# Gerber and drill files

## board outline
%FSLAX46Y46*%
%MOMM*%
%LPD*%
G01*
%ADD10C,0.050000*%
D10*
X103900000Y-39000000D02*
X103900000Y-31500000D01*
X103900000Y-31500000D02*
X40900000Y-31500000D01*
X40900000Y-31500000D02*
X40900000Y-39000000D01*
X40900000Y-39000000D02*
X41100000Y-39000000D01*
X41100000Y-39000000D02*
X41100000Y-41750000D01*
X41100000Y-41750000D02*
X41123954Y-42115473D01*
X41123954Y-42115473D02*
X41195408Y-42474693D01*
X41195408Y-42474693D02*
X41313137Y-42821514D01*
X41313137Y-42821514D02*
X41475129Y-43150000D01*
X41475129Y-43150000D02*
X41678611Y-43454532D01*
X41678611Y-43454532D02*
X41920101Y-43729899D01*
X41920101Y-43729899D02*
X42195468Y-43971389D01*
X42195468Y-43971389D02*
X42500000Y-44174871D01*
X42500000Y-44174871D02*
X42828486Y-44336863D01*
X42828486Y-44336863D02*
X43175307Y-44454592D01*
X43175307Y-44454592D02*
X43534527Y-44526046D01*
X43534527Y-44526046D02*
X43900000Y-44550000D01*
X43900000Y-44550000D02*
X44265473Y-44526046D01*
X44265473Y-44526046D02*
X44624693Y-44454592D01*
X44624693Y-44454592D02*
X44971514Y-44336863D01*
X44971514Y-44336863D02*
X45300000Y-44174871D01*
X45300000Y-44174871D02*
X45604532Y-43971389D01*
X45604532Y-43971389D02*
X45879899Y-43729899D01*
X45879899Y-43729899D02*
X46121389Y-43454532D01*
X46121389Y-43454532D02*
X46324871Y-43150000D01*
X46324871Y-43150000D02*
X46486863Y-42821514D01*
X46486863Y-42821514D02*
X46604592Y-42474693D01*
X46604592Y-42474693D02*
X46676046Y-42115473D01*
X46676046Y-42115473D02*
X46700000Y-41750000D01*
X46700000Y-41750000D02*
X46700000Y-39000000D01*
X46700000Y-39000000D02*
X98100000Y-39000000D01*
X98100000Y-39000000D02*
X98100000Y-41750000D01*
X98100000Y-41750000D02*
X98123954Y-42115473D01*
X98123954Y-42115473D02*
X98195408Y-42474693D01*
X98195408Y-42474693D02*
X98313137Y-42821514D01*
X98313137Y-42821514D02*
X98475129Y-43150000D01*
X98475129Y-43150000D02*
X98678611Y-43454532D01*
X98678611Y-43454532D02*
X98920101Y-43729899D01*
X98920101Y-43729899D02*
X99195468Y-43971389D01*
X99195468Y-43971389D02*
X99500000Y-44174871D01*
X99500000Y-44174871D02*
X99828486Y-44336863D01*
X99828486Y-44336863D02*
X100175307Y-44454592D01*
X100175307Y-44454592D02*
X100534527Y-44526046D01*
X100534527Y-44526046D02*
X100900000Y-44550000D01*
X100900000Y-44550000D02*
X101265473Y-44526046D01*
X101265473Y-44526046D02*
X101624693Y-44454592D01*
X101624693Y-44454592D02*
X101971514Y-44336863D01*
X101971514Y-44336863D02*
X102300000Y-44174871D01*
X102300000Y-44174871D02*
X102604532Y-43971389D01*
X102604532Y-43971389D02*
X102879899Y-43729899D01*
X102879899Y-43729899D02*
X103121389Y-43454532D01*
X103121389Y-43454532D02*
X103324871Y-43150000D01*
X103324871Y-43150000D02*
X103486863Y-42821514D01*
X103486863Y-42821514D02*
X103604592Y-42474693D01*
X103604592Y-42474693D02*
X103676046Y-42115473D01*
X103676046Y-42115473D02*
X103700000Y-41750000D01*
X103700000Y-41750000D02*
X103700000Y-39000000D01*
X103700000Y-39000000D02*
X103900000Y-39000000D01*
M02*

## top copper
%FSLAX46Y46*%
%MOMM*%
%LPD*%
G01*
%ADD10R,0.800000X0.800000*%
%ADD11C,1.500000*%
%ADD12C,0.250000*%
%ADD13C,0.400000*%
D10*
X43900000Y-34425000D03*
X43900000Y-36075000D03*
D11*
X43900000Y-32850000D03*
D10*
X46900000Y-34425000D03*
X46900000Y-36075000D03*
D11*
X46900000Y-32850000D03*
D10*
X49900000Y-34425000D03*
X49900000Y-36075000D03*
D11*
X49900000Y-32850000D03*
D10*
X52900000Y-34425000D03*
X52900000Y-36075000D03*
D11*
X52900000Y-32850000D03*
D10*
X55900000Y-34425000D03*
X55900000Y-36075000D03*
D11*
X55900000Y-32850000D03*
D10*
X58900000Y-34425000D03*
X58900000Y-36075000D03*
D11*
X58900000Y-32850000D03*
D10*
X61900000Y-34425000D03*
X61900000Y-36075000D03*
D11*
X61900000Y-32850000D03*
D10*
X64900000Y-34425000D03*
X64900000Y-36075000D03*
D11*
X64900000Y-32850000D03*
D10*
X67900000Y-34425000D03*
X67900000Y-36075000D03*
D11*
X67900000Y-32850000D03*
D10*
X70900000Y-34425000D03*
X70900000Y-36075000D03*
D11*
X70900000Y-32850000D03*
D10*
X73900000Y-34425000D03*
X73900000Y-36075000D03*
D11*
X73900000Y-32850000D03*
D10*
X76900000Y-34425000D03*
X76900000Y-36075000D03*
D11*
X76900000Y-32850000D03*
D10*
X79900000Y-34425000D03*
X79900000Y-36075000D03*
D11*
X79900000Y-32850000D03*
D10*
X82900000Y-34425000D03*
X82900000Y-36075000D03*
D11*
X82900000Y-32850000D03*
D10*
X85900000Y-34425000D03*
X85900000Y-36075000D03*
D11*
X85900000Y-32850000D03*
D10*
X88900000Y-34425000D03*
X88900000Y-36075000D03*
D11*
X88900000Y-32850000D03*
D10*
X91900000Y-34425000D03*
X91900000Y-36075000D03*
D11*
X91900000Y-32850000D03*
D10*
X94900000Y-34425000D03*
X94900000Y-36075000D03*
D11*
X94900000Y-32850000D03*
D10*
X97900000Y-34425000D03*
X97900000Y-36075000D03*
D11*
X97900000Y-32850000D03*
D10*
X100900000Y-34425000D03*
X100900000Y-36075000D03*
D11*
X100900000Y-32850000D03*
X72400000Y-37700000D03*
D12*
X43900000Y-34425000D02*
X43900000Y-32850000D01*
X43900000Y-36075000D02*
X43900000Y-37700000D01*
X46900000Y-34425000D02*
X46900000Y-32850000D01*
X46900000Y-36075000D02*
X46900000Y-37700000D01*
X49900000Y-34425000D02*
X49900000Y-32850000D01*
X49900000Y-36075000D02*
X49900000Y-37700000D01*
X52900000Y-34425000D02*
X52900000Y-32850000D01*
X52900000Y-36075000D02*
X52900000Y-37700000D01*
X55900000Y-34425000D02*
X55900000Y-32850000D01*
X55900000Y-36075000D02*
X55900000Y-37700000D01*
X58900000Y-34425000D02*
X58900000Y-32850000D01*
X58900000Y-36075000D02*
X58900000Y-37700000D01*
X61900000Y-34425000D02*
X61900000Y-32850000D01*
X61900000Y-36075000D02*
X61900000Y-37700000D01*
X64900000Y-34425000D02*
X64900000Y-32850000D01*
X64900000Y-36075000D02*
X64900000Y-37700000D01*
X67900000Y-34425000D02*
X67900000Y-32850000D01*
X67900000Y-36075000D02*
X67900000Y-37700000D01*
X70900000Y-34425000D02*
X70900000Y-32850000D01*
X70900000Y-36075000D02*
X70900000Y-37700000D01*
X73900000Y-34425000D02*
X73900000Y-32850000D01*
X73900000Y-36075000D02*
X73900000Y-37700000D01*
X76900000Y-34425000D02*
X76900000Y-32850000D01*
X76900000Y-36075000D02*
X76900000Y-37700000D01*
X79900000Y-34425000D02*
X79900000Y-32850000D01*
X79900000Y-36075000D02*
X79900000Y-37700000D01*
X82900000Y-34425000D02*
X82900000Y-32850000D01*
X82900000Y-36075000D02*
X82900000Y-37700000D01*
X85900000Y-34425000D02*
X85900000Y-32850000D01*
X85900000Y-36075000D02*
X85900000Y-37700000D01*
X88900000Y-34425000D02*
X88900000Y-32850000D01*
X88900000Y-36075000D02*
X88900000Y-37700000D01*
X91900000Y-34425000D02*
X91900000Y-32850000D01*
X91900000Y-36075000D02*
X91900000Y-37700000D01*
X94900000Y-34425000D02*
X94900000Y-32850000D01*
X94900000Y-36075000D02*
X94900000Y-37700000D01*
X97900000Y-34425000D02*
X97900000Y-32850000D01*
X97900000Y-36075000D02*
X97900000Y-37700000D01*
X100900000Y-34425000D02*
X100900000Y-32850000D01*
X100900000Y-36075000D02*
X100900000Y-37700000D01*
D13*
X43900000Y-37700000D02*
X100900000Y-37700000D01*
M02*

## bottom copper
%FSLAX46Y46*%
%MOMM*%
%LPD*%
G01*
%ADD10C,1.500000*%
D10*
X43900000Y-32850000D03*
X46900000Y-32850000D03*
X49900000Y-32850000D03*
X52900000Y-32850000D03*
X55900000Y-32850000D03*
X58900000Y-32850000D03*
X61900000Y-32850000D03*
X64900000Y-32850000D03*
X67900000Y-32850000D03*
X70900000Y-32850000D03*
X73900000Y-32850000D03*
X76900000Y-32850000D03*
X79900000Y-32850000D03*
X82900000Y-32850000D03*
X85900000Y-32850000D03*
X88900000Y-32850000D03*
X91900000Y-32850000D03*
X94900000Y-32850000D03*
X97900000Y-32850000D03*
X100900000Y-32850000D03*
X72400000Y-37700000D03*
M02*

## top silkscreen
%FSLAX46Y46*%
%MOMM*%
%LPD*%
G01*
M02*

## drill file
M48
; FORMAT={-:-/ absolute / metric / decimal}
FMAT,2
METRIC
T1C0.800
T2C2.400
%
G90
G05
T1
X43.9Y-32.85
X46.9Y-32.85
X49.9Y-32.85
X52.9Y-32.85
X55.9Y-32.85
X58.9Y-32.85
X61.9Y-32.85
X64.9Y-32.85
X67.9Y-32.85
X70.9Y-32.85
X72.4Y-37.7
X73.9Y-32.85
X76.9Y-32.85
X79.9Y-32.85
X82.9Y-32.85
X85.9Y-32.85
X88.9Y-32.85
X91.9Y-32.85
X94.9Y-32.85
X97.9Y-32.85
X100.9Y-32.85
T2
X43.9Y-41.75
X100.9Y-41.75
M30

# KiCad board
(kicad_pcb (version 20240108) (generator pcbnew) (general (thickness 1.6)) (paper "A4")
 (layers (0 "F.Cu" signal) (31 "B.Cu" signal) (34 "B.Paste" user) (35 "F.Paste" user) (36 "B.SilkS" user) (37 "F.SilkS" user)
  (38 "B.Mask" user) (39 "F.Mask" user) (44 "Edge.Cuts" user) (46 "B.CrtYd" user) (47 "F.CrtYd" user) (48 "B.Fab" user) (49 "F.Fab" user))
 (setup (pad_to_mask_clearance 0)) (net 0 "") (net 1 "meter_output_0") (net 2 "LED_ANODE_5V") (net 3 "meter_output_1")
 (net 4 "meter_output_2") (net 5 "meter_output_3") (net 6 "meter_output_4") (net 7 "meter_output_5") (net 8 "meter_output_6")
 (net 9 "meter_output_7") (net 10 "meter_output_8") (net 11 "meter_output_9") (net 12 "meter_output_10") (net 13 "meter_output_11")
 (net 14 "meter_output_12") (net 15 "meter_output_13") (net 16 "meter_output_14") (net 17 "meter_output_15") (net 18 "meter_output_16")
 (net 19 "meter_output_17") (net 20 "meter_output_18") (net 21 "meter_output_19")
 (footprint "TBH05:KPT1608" (layer "F.Cu") (at 43.9 35.25)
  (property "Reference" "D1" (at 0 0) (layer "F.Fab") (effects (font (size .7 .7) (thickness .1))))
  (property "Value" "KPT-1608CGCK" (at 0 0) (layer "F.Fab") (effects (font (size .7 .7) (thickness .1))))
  (pad "1" smd rect (at 0 -.825) (size .8 .8) (layers "F.Cu" "F.Paste" "F.Mask") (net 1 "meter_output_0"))
  (pad "2" smd rect (at 0 .825) (size .8 .8) (layers "F.Cu" "F.Paste" "F.Mask") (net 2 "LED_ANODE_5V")))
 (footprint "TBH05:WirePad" (layer "F.Cu") (at 43.9 32.85)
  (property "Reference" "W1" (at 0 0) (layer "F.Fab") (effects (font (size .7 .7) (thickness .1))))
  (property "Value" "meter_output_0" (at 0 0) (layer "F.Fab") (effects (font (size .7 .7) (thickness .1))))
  (pad "1" thru_hole circle (at 0 0) (size 1.5 1.5) (drill .8) (layers "*.Cu" "*.Mask") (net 1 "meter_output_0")))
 (segment (start 43.9 34.425) (end 43.9 32.85) (width 0.25) (layer "F.Cu") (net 1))
 (segment (start 43.9 36.075) (end 43.9 37.7) (width 0.25) (layer "F.Cu") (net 2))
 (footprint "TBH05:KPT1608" (layer "F.Cu") (at 46.9 35.25)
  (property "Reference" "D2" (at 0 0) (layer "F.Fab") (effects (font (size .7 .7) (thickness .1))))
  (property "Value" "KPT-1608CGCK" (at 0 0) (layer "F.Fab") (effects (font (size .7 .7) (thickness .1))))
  (pad "1" smd rect (at 0 -.825) (size .8 .8) (layers "F.Cu" "F.Paste" "F.Mask") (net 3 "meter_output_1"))
  (pad "2" smd rect (at 0 .825) (size .8 .8) (layers "F.Cu" "F.Paste" "F.Mask") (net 2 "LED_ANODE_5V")))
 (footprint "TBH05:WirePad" (layer "F.Cu") (at 46.9 32.85)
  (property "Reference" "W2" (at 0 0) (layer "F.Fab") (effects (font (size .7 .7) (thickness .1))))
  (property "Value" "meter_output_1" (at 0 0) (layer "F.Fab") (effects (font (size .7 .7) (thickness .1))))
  (pad "1" thru_hole circle (at 0 0) (size 1.5 1.5) (drill .8) (layers "*.Cu" "*.Mask") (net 3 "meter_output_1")))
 (segment (start 46.9 34.425) (end 46.9 32.85) (width 0.25) (layer "F.Cu") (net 3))
 (segment (start 46.9 36.075) (end 46.9 37.7) (width 0.25) (layer "F.Cu") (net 2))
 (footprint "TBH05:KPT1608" (layer "F.Cu") (at 49.9 35.25)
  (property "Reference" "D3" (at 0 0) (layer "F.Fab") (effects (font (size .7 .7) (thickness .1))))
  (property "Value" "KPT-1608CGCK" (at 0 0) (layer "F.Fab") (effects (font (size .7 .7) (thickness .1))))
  (pad "1" smd rect (at 0 -.825) (size .8 .8) (layers "F.Cu" "F.Paste" "F.Mask") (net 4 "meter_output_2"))
  (pad "2" smd rect (at 0 .825) (size .8 .8) (layers "F.Cu" "F.Paste" "F.Mask") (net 2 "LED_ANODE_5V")))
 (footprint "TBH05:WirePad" (layer "F.Cu") (at 49.9 32.85)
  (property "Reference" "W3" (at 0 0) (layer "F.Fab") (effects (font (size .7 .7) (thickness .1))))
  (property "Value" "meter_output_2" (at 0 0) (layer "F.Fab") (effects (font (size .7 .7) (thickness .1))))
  (pad "1" thru_hole circle (at 0 0) (size 1.5 1.5) (drill .8) (layers "*.Cu" "*.Mask") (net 4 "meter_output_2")))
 (segment (start 49.9 34.425) (end 49.9 32.85) (width 0.25) (layer "F.Cu") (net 4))
 (segment (start 49.9 36.075) (end 49.9 37.7) (width 0.25) (layer "F.Cu") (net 2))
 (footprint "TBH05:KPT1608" (layer "F.Cu") (at 52.9 35.25)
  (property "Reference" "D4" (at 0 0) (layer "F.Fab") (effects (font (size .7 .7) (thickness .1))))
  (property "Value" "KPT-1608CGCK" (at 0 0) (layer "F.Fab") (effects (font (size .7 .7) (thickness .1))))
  (pad "1" smd rect (at 0 -.825) (size .8 .8) (layers "F.Cu" "F.Paste" "F.Mask") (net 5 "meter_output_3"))
  (pad "2" smd rect (at 0 .825) (size .8 .8) (layers "F.Cu" "F.Paste" "F.Mask") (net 2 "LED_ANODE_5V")))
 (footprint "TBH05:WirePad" (layer "F.Cu") (at 52.9 32.85)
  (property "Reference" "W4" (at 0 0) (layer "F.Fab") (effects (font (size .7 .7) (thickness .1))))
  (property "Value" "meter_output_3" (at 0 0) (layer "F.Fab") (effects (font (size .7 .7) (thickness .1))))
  (pad "1" thru_hole circle (at 0 0) (size 1.5 1.5) (drill .8) (layers "*.Cu" "*.Mask") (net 5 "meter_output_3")))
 (segment (start 52.9 34.425) (end 52.9 32.85) (width 0.25) (layer "F.Cu") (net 5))
 (segment (start 52.9 36.075) (end 52.9 37.7) (width 0.25) (layer "F.Cu") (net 2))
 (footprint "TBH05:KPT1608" (layer "F.Cu") (at 55.9 35.25)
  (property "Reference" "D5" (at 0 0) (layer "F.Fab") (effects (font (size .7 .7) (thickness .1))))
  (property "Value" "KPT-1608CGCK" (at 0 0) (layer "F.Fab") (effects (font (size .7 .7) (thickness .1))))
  (pad "1" smd rect (at 0 -.825) (size .8 .8) (layers "F.Cu" "F.Paste" "F.Mask") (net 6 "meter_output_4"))
  (pad "2" smd rect (at 0 .825) (size .8 .8) (layers "F.Cu" "F.Paste" "F.Mask") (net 2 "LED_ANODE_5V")))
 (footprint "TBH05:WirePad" (layer "F.Cu") (at 55.9 32.85)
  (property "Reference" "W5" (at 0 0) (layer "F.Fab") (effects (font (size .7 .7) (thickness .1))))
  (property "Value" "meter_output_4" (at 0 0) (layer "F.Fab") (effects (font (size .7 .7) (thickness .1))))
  (pad "1" thru_hole circle (at 0 0) (size 1.5 1.5) (drill .8) (layers "*.Cu" "*.Mask") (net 6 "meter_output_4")))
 (segment (start 55.9 34.425) (end 55.9 32.85) (width 0.25) (layer "F.Cu") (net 6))
 (segment (start 55.9 36.075) (end 55.9 37.7) (width 0.25) (layer "F.Cu") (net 2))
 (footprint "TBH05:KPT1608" (layer "F.Cu") (at 58.9 35.25)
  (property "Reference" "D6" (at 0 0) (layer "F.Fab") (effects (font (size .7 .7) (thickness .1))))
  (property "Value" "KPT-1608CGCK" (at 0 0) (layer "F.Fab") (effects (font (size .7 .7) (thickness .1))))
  (pad "1" smd rect (at 0 -.825) (size .8 .8) (layers "F.Cu" "F.Paste" "F.Mask") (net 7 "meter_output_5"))
  (pad "2" smd rect (at 0 .825) (size .8 .8) (layers "F.Cu" "F.Paste" "F.Mask") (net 2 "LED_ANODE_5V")))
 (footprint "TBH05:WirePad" (layer "F.Cu") (at 58.9 32.85)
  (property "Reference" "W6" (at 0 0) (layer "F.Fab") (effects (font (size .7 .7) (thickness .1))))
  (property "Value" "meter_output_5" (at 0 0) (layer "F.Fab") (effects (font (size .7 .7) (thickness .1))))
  (pad "1" thru_hole circle (at 0 0) (size 1.5 1.5) (drill .8) (layers "*.Cu" "*.Mask") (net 7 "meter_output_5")))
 (segment (start 58.9 34.425) (end 58.9 32.85) (width 0.25) (layer "F.Cu") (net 7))
 (segment (start 58.9 36.075) (end 58.9 37.7) (width 0.25) (layer "F.Cu") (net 2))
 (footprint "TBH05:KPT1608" (layer "F.Cu") (at 61.9 35.25)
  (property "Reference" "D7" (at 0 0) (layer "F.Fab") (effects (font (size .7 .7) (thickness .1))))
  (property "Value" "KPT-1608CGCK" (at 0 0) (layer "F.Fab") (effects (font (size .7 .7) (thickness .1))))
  (pad "1" smd rect (at 0 -.825) (size .8 .8) (layers "F.Cu" "F.Paste" "F.Mask") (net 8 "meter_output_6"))
  (pad "2" smd rect (at 0 .825) (size .8 .8) (layers "F.Cu" "F.Paste" "F.Mask") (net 2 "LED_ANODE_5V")))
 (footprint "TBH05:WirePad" (layer "F.Cu") (at 61.9 32.85)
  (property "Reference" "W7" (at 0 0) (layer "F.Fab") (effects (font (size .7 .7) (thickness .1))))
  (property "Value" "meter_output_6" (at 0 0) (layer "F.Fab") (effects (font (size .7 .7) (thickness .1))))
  (pad "1" thru_hole circle (at 0 0) (size 1.5 1.5) (drill .8) (layers "*.Cu" "*.Mask") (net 8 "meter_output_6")))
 (segment (start 61.9 34.425) (end 61.9 32.85) (width 0.25) (layer "F.Cu") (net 8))
 (segment (start 61.9 36.075) (end 61.9 37.7) (width 0.25) (layer "F.Cu") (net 2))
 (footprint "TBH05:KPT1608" (layer "F.Cu") (at 64.9 35.25)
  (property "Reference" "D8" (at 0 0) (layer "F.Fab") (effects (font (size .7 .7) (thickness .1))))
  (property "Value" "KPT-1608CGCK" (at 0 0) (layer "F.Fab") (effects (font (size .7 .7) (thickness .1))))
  (pad "1" smd rect (at 0 -.825) (size .8 .8) (layers "F.Cu" "F.Paste" "F.Mask") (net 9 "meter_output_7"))
  (pad "2" smd rect (at 0 .825) (size .8 .8) (layers "F.Cu" "F.Paste" "F.Mask") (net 2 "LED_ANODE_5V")))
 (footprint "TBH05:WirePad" (layer "F.Cu") (at 64.9 32.85)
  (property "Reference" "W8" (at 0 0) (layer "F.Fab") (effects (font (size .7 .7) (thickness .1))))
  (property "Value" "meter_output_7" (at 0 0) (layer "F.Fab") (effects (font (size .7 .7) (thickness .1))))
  (pad "1" thru_hole circle (at 0 0) (size 1.5 1.5) (drill .8) (layers "*.Cu" "*.Mask") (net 9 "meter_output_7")))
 (segment (start 64.9 34.425) (end 64.9 32.85) (width 0.25) (layer "F.Cu") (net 9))
 (segment (start 64.9 36.075) (end 64.9 37.7) (width 0.25) (layer "F.Cu") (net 2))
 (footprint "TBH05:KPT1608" (layer "F.Cu") (at 67.9 35.25)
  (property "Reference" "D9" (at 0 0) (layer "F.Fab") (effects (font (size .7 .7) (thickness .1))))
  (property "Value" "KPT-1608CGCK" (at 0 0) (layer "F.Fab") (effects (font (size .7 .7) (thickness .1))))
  (pad "1" smd rect (at 0 -.825) (size .8 .8) (layers "F.Cu" "F.Paste" "F.Mask") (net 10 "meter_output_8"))
  (pad "2" smd rect (at 0 .825) (size .8 .8) (layers "F.Cu" "F.Paste" "F.Mask") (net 2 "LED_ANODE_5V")))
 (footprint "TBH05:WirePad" (layer "F.Cu") (at 67.9 32.85)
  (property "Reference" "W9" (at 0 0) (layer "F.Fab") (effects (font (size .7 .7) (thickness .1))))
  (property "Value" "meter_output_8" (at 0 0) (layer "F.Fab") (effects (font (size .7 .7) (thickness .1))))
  (pad "1" thru_hole circle (at 0 0) (size 1.5 1.5) (drill .8) (layers "*.Cu" "*.Mask") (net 10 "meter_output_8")))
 (segment (start 67.9 34.425) (end 67.9 32.85) (width 0.25) (layer "F.Cu") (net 10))
 (segment (start 67.9 36.075) (end 67.9 37.7) (width 0.25) (layer "F.Cu") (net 2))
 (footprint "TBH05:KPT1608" (layer "F.Cu") (at 70.9 35.25)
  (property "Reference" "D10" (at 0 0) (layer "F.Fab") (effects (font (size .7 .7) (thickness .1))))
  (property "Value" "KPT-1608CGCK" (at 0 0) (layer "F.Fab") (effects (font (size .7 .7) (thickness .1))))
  (pad "1" smd rect (at 0 -.825) (size .8 .8) (layers "F.Cu" "F.Paste" "F.Mask") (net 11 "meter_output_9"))
  (pad "2" smd rect (at 0 .825) (size .8 .8) (layers "F.Cu" "F.Paste" "F.Mask") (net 2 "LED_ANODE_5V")))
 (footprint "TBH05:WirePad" (layer "F.Cu") (at 70.9 32.85)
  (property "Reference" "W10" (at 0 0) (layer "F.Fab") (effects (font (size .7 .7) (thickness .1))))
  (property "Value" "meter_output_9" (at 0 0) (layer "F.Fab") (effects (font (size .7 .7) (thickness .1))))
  (pad "1" thru_hole circle (at 0 0) (size 1.5 1.5) (drill .8) (layers "*.Cu" "*.Mask") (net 11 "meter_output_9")))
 (segment (start 70.9 34.425) (end 70.9 32.85) (width 0.25) (layer "F.Cu") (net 11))
 (segment (start 70.9 36.075) (end 70.9 37.7) (width 0.25) (layer "F.Cu") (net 2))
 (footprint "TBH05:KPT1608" (layer "F.Cu") (at 73.9 35.25)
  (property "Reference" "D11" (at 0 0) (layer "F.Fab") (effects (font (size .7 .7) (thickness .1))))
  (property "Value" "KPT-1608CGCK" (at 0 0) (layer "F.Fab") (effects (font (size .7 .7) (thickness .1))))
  (pad "1" smd rect (at 0 -.825) (size .8 .8) (layers "F.Cu" "F.Paste" "F.Mask") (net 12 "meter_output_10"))
  (pad "2" smd rect (at 0 .825) (size .8 .8) (layers "F.Cu" "F.Paste" "F.Mask") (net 2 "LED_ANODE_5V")))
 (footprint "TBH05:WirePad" (layer "F.Cu") (at 73.9 32.85)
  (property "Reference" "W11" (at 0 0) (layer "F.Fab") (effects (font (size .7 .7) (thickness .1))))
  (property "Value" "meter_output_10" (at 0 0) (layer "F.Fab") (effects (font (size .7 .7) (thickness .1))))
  (pad "1" thru_hole circle (at 0 0) (size 1.5 1.5) (drill .8) (layers "*.Cu" "*.Mask") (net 12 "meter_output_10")))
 (segment (start 73.9 34.425) (end 73.9 32.85) (width 0.25) (layer "F.Cu") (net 12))
 (segment (start 73.9 36.075) (end 73.9 37.7) (width 0.25) (layer "F.Cu") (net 2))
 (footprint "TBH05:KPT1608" (layer "F.Cu") (at 76.9 35.25)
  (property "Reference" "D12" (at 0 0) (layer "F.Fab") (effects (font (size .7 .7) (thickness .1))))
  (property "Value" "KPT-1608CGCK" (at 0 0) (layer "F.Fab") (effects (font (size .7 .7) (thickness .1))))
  (pad "1" smd rect (at 0 -.825) (size .8 .8) (layers "F.Cu" "F.Paste" "F.Mask") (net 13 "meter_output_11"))
  (pad "2" smd rect (at 0 .825) (size .8 .8) (layers "F.Cu" "F.Paste" "F.Mask") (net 2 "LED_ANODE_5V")))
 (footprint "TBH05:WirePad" (layer "F.Cu") (at 76.9 32.85)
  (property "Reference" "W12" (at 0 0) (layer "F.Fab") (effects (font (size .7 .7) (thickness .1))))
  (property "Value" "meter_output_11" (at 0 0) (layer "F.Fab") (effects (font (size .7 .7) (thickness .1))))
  (pad "1" thru_hole circle (at 0 0) (size 1.5 1.5) (drill .8) (layers "*.Cu" "*.Mask") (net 13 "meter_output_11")))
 (segment (start 76.9 34.425) (end 76.9 32.85) (width 0.25) (layer "F.Cu") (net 13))
 (segment (start 76.9 36.075) (end 76.9 37.7) (width 0.25) (layer "F.Cu") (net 2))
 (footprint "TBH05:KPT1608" (layer "F.Cu") (at 79.9 35.25)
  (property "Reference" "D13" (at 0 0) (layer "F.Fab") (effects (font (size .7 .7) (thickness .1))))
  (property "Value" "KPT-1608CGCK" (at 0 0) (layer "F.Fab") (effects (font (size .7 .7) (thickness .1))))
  (pad "1" smd rect (at 0 -.825) (size .8 .8) (layers "F.Cu" "F.Paste" "F.Mask") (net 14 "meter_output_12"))
  (pad "2" smd rect (at 0 .825) (size .8 .8) (layers "F.Cu" "F.Paste" "F.Mask") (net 2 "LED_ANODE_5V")))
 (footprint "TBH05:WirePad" (layer "F.Cu") (at 79.9 32.85)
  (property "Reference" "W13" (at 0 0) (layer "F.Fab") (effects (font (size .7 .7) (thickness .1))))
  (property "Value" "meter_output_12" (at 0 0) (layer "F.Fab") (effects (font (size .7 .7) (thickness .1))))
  (pad "1" thru_hole circle (at 0 0) (size 1.5 1.5) (drill .8) (layers "*.Cu" "*.Mask") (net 14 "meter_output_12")))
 (segment (start 79.9 34.425) (end 79.9 32.85) (width 0.25) (layer "F.Cu") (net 14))
 (segment (start 79.9 36.075) (end 79.9 37.7) (width 0.25) (layer "F.Cu") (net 2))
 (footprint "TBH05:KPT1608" (layer "F.Cu") (at 82.9 35.25)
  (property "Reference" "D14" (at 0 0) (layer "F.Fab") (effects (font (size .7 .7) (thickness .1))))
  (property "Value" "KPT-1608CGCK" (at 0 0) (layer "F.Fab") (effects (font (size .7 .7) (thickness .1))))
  (pad "1" smd rect (at 0 -.825) (size .8 .8) (layers "F.Cu" "F.Paste" "F.Mask") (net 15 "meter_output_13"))
  (pad "2" smd rect (at 0 .825) (size .8 .8) (layers "F.Cu" "F.Paste" "F.Mask") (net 2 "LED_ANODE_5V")))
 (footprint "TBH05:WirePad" (layer "F.Cu") (at 82.9 32.85)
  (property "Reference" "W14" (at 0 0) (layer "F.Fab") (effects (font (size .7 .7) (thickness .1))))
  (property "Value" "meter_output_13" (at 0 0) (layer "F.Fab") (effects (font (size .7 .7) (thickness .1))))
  (pad "1" thru_hole circle (at 0 0) (size 1.5 1.5) (drill .8) (layers "*.Cu" "*.Mask") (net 15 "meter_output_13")))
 (segment (start 82.9 34.425) (end 82.9 32.85) (width 0.25) (layer "F.Cu") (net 15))
 (segment (start 82.9 36.075) (end 82.9 37.7) (width 0.25) (layer "F.Cu") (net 2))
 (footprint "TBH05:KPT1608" (layer "F.Cu") (at 85.9 35.25)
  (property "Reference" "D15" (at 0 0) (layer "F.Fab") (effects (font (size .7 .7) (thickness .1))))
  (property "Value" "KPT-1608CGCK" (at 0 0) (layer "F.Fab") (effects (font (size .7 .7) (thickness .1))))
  (pad "1" smd rect (at 0 -.825) (size .8 .8) (layers "F.Cu" "F.Paste" "F.Mask") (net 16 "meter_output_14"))
  (pad "2" smd rect (at 0 .825) (size .8 .8) (layers "F.Cu" "F.Paste" "F.Mask") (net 2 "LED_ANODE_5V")))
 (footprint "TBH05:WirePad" (layer "F.Cu") (at 85.9 32.85)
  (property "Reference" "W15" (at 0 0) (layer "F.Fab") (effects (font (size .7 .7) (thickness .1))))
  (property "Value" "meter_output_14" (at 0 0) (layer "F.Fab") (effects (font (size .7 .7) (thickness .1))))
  (pad "1" thru_hole circle (at 0 0) (size 1.5 1.5) (drill .8) (layers "*.Cu" "*.Mask") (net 16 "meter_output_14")))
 (segment (start 85.9 34.425) (end 85.9 32.85) (width 0.25) (layer "F.Cu") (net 16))
 (segment (start 85.9 36.075) (end 85.9 37.7) (width 0.25) (layer "F.Cu") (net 2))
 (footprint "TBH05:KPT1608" (layer "F.Cu") (at 88.9 35.25)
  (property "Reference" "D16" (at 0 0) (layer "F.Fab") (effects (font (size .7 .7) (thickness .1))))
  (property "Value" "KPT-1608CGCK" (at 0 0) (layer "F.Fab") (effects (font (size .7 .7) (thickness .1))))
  (pad "1" smd rect (at 0 -.825) (size .8 .8) (layers "F.Cu" "F.Paste" "F.Mask") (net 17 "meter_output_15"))
  (pad "2" smd rect (at 0 .825) (size .8 .8) (layers "F.Cu" "F.Paste" "F.Mask") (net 2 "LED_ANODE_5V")))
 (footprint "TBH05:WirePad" (layer "F.Cu") (at 88.9 32.85)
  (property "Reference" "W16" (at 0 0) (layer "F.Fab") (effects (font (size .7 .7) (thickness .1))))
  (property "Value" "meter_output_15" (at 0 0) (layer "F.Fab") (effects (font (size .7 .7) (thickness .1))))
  (pad "1" thru_hole circle (at 0 0) (size 1.5 1.5) (drill .8) (layers "*.Cu" "*.Mask") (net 17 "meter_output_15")))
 (segment (start 88.9 34.425) (end 88.9 32.85) (width 0.25) (layer "F.Cu") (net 17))
 (segment (start 88.9 36.075) (end 88.9 37.7) (width 0.25) (layer "F.Cu") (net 2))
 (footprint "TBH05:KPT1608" (layer "F.Cu") (at 91.9 35.25)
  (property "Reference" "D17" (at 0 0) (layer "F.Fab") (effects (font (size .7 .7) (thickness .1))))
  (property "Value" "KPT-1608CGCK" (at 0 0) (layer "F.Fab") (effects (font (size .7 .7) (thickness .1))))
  (pad "1" smd rect (at 0 -.825) (size .8 .8) (layers "F.Cu" "F.Paste" "F.Mask") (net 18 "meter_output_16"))
  (pad "2" smd rect (at 0 .825) (size .8 .8) (layers "F.Cu" "F.Paste" "F.Mask") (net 2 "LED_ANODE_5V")))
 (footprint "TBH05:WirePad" (layer "F.Cu") (at 91.9 32.85)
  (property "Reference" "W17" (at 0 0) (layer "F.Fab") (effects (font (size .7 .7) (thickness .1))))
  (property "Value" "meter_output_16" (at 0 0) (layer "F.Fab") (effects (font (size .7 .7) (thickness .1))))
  (pad "1" thru_hole circle (at 0 0) (size 1.5 1.5) (drill .8) (layers "*.Cu" "*.Mask") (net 18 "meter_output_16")))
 (segment (start 91.9 34.425) (end 91.9 32.85) (width 0.25) (layer "F.Cu") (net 18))
 (segment (start 91.9 36.075) (end 91.9 37.7) (width 0.25) (layer "F.Cu") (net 2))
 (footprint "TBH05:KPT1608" (layer "F.Cu") (at 94.9 35.25)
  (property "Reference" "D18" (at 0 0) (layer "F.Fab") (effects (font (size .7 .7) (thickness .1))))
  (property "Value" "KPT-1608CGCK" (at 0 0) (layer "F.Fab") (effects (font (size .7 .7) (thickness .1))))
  (pad "1" smd rect (at 0 -.825) (size .8 .8) (layers "F.Cu" "F.Paste" "F.Mask") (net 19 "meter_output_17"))
  (pad "2" smd rect (at 0 .825) (size .8 .8) (layers "F.Cu" "F.Paste" "F.Mask") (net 2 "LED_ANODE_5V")))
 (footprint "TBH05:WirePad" (layer "F.Cu") (at 94.9 32.85)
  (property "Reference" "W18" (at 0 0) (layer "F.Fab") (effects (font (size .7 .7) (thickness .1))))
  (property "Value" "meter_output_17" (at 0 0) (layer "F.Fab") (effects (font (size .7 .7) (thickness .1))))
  (pad "1" thru_hole circle (at 0 0) (size 1.5 1.5) (drill .8) (layers "*.Cu" "*.Mask") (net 19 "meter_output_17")))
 (segment (start 94.9 34.425) (end 94.9 32.85) (width 0.25) (layer "F.Cu") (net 19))
 (segment (start 94.9 36.075) (end 94.9 37.7) (width 0.25) (layer "F.Cu") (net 2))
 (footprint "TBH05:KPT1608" (layer "F.Cu") (at 97.9 35.25)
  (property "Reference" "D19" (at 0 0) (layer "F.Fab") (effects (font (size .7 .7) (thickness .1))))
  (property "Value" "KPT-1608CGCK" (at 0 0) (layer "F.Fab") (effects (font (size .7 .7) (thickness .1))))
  (pad "1" smd rect (at 0 -.825) (size .8 .8) (layers "F.Cu" "F.Paste" "F.Mask") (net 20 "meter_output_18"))
  (pad "2" smd rect (at 0 .825) (size .8 .8) (layers "F.Cu" "F.Paste" "F.Mask") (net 2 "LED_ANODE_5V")))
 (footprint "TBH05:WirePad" (layer "F.Cu") (at 97.9 32.85)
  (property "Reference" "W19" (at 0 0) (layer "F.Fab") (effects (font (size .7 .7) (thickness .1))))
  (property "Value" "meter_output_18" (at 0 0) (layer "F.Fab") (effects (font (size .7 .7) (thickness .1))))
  (pad "1" thru_hole circle (at 0 0) (size 1.5 1.5) (drill .8) (layers "*.Cu" "*.Mask") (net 20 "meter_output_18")))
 (segment (start 97.9 34.425) (end 97.9 32.85) (width 0.25) (layer "F.Cu") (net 20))
 (segment (start 97.9 36.075) (end 97.9 37.7) (width 0.25) (layer "F.Cu") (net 2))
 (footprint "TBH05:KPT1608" (layer "F.Cu") (at 100.9 35.25)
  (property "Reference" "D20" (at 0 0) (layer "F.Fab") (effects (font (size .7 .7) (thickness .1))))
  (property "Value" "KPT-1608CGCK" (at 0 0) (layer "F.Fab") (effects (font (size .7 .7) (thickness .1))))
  (pad "1" smd rect (at 0 -.825) (size .8 .8) (layers "F.Cu" "F.Paste" "F.Mask") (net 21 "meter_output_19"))
  (pad "2" smd rect (at 0 .825) (size .8 .8) (layers "F.Cu" "F.Paste" "F.Mask") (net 2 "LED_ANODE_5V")))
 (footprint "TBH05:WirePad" (layer "F.Cu") (at 100.9 32.85)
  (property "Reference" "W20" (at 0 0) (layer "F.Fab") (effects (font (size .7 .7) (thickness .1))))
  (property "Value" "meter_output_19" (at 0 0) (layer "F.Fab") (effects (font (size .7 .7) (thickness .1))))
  (pad "1" thru_hole circle (at 0 0) (size 1.5 1.5) (drill .8) (layers "*.Cu" "*.Mask") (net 21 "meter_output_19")))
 (segment (start 100.9 34.425) (end 100.9 32.85) (width 0.25) (layer "F.Cu") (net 21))
 (segment (start 100.9 36.075) (end 100.9 37.7) (width 0.25) (layer "F.Cu") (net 2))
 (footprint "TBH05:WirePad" (layer "F.Cu") (at 72.4 37.7)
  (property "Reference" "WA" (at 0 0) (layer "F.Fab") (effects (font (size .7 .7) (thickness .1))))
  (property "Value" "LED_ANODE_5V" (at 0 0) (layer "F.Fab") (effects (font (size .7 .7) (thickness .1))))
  (pad "1" thru_hole circle (at 0 0) (size 1.5 1.5) (drill .8) (layers "*.Cu" "*.Mask") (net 2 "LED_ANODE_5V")))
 (segment (start 43.9 37.7) (end 100.9 37.7) (width 0.4) (layer "F.Cu") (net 2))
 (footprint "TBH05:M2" (layer "F.Cu") (at 43.9 41.75)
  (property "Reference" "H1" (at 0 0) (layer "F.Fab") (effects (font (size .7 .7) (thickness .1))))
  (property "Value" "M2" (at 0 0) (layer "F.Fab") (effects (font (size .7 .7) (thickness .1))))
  (pad "" np_thru_hole circle (at 0 0) (size 2.4 2.4) (drill 2.4) (layers "*.Cu" "*.Mask")))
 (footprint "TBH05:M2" (layer "F.Cu") (at 100.9 41.75)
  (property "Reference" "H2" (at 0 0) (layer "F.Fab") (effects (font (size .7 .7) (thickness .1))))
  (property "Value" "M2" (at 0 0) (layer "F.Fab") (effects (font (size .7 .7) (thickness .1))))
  (pad "" np_thru_hole circle (at 0 0) (size 2.4 2.4) (drill 2.4) (layers "*.Cu" "*.Mask")))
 (gr_line (start 103.9 39.0) (end 103.9 31.5) (stroke (width .05) (type default)) (layer "Edge.Cuts"))
 (gr_line (start 103.9 31.5) (end 40.9 31.5) (stroke (width .05) (type default)) (layer "Edge.Cuts"))
 (gr_line (start 40.9 31.5) (end 40.9 39.0) (stroke (width .05) (type default)) (layer "Edge.Cuts"))
 (gr_line (start 40.9 39.0) (end 41.1 39.0) (stroke (width .05) (type default)) (layer "Edge.Cuts"))
 (gr_line (start 41.1 39.0) (end 41.1 41.75) (stroke (width .05) (type default)) (layer "Edge.Cuts"))
 (gr_line (start 41.1 41.75) (end 41.123954 42.115473) (stroke (width .05) (type default)) (layer "Edge.Cuts"))
 (gr_line (start 41.123954 42.115473) (end 41.195408 42.474693) (stroke (width .05) (type default)) (layer "Edge.Cuts"))
 (gr_line (start 41.195408 42.474693) (end 41.313137 42.821514) (stroke (width .05) (type default)) (layer "Edge.Cuts"))
 (gr_line (start 41.313137 42.821514) (end 41.475129 43.15) (stroke (width .05) (type default)) (layer "Edge.Cuts"))
 (gr_line (start 41.475129 43.15) (end 41.678611 43.454532) (stroke (width .05) (type default)) (layer "Edge.Cuts"))
 (gr_line (start 41.678611 43.454532) (end 41.920101 43.729899) (stroke (width .05) (type default)) (layer "Edge.Cuts"))
 (gr_line (start 41.920101 43.729899) (end 42.195468 43.971389) (stroke (width .05) (type default)) (layer "Edge.Cuts"))
 (gr_line (start 42.195468 43.971389) (end 42.5 44.174871) (stroke (width .05) (type default)) (layer "Edge.Cuts"))
 (gr_line (start 42.5 44.174871) (end 42.828486 44.336863) (stroke (width .05) (type default)) (layer "Edge.Cuts"))
 (gr_line (start 42.828486 44.336863) (end 43.175307 44.454592) (stroke (width .05) (type default)) (layer "Edge.Cuts"))
 (gr_line (start 43.175307 44.454592) (end 43.534527 44.526046) (stroke (width .05) (type default)) (layer "Edge.Cuts"))
 (gr_line (start 43.534527 44.526046) (end 43.9 44.55) (stroke (width .05) (type default)) (layer "Edge.Cuts"))
 (gr_line (start 43.9 44.55) (end 44.265473 44.526046) (stroke (width .05) (type default)) (layer "Edge.Cuts"))
 (gr_line (start 44.265473 44.526046) (end 44.624693 44.454592) (stroke (width .05) (type default)) (layer "Edge.Cuts"))
 (gr_line (start 44.624693 44.454592) (end 44.971514 44.336863) (stroke (width .05) (type default)) (layer "Edge.Cuts"))
 (gr_line (start 44.971514 44.336863) (end 45.3 44.174871) (stroke (width .05) (type default)) (layer "Edge.Cuts"))
 (gr_line (start 45.3 44.174871) (end 45.604532 43.971389) (stroke (width .05) (type default)) (layer "Edge.Cuts"))
 (gr_line (start 45.604532 43.971389) (end 45.879899 43.729899) (stroke (width .05) (type default)) (layer "Edge.Cuts"))
 (gr_line (start 45.879899 43.729899) (end 46.121389 43.454532) (stroke (width .05) (type default)) (layer "Edge.Cuts"))
 (gr_line (start 46.121389 43.454532) (end 46.324871 43.15) (stroke (width .05) (type default)) (layer "Edge.Cuts"))
 (gr_line (start 46.324871 43.15) (end 46.486863 42.821514) (stroke (width .05) (type default)) (layer "Edge.Cuts"))
 (gr_line (start 46.486863 42.821514) (end 46.604592 42.474693) (stroke (width .05) (type default)) (layer "Edge.Cuts"))
 (gr_line (start 46.604592 42.474693) (end 46.676046 42.115473) (stroke (width .05) (type default)) (layer "Edge.Cuts"))
 (gr_line (start 46.676046 42.115473) (end 46.7 41.75) (stroke (width .05) (type default)) (layer "Edge.Cuts"))
 (gr_line (start 46.7 41.75) (end 46.7 39.0) (stroke (width .05) (type default)) (layer "Edge.Cuts"))
 (gr_line (start 46.7 39.0) (end 98.1 39.0) (stroke (width .05) (type default)) (layer "Edge.Cuts"))
 (gr_line (start 98.1 39.0) (end 98.1 41.75) (stroke (width .05) (type default)) (layer "Edge.Cuts"))
 (gr_line (start 98.1 41.75) (end 98.123954 42.115473) (stroke (width .05) (type default)) (layer "Edge.Cuts"))
 (gr_line (start 98.123954 42.115473) (end 98.195408 42.474693) (stroke (width .05) (type default)) (layer "Edge.Cuts"))
 (gr_line (start 98.195408 42.474693) (end 98.313137 42.821514) (stroke (width .05) (type default)) (layer "Edge.Cuts"))
 (gr_line (start 98.313137 42.821514) (end 98.475129 43.15) (stroke (width .05) (type default)) (layer "Edge.Cuts"))
 (gr_line (start 98.475129 43.15) (end 98.678611 43.454532) (stroke (width .05) (type default)) (layer "Edge.Cuts"))
 (gr_line (start 98.678611 43.454532) (end 98.920101 43.729899) (stroke (width .05) (type default)) (layer "Edge.Cuts"))
 (gr_line (start 98.920101 43.729899) (end 99.195468 43.971389) (stroke (width .05) (type default)) (layer "Edge.Cuts"))
 (gr_line (start 99.195468 43.971389) (end 99.5 44.174871) (stroke (width .05) (type default)) (layer "Edge.Cuts"))
 (gr_line (start 99.5 44.174871) (end 99.828486 44.336863) (stroke (width .05) (type default)) (layer "Edge.Cuts"))
 (gr_line (start 99.828486 44.336863) (end 100.175307 44.454592) (stroke (width .05) (type default)) (layer "Edge.Cuts"))
 (gr_line (start 100.175307 44.454592) (end 100.534527 44.526046) (stroke (width .05) (type default)) (layer "Edge.Cuts"))
 (gr_line (start 100.534527 44.526046) (end 100.9 44.55) (stroke (width .05) (type default)) (layer "Edge.Cuts"))
 (gr_line (start 100.9 44.55) (end 101.265473 44.526046) (stroke (width .05) (type default)) (layer "Edge.Cuts"))
 (gr_line (start 101.265473 44.526046) (end 101.624693 44.454592) (stroke (width .05) (type default)) (layer "Edge.Cuts"))
 (gr_line (start 101.624693 44.454592) (end 101.971514 44.336863) (stroke (width .05) (type default)) (layer "Edge.Cuts"))
 (gr_line (start 101.971514 44.336863) (end 102.3 44.174871) (stroke (width .05) (type default)) (layer "Edge.Cuts"))
 (gr_line (start 102.3 44.174871) (end 102.604532 43.971389) (stroke (width .05) (type default)) (layer "Edge.Cuts"))
 (gr_line (start 102.604532 43.971389) (end 102.879899 43.729899) (stroke (width .05) (type default)) (layer "Edge.Cuts"))
 (gr_line (start 102.879899 43.729899) (end 103.121389 43.454532) (stroke (width .05) (type default)) (layer "Edge.Cuts"))
 (gr_line (start 103.121389 43.454532) (end 103.324871 43.15) (stroke (width .05) (type default)) (layer "Edge.Cuts"))
 (gr_line (start 103.324871 43.15) (end 103.486863 42.821514) (stroke (width .05) (type default)) (layer "Edge.Cuts"))
 (gr_line (start 103.486863 42.821514) (end 103.604592 42.474693) (stroke (width .05) (type default)) (layer "Edge.Cuts"))
 (gr_line (start 103.604592 42.474693) (end 103.676046 42.115473) (stroke (width .05) (type default)) (layer "Edge.Cuts"))
 (gr_line (start 103.676046 42.115473) (end 103.7 41.75) (stroke (width .05) (type default)) (layer "Edge.Cuts"))
 (gr_line (start 103.7 41.75) (end 103.7 39.0) (stroke (width .05) (type default)) (layer "Edge.Cuts"))
 (gr_line (start 103.7 39.0) (end 103.9 39.0) (stroke (width .05) (type default)) (layer "Edge.Cuts")))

